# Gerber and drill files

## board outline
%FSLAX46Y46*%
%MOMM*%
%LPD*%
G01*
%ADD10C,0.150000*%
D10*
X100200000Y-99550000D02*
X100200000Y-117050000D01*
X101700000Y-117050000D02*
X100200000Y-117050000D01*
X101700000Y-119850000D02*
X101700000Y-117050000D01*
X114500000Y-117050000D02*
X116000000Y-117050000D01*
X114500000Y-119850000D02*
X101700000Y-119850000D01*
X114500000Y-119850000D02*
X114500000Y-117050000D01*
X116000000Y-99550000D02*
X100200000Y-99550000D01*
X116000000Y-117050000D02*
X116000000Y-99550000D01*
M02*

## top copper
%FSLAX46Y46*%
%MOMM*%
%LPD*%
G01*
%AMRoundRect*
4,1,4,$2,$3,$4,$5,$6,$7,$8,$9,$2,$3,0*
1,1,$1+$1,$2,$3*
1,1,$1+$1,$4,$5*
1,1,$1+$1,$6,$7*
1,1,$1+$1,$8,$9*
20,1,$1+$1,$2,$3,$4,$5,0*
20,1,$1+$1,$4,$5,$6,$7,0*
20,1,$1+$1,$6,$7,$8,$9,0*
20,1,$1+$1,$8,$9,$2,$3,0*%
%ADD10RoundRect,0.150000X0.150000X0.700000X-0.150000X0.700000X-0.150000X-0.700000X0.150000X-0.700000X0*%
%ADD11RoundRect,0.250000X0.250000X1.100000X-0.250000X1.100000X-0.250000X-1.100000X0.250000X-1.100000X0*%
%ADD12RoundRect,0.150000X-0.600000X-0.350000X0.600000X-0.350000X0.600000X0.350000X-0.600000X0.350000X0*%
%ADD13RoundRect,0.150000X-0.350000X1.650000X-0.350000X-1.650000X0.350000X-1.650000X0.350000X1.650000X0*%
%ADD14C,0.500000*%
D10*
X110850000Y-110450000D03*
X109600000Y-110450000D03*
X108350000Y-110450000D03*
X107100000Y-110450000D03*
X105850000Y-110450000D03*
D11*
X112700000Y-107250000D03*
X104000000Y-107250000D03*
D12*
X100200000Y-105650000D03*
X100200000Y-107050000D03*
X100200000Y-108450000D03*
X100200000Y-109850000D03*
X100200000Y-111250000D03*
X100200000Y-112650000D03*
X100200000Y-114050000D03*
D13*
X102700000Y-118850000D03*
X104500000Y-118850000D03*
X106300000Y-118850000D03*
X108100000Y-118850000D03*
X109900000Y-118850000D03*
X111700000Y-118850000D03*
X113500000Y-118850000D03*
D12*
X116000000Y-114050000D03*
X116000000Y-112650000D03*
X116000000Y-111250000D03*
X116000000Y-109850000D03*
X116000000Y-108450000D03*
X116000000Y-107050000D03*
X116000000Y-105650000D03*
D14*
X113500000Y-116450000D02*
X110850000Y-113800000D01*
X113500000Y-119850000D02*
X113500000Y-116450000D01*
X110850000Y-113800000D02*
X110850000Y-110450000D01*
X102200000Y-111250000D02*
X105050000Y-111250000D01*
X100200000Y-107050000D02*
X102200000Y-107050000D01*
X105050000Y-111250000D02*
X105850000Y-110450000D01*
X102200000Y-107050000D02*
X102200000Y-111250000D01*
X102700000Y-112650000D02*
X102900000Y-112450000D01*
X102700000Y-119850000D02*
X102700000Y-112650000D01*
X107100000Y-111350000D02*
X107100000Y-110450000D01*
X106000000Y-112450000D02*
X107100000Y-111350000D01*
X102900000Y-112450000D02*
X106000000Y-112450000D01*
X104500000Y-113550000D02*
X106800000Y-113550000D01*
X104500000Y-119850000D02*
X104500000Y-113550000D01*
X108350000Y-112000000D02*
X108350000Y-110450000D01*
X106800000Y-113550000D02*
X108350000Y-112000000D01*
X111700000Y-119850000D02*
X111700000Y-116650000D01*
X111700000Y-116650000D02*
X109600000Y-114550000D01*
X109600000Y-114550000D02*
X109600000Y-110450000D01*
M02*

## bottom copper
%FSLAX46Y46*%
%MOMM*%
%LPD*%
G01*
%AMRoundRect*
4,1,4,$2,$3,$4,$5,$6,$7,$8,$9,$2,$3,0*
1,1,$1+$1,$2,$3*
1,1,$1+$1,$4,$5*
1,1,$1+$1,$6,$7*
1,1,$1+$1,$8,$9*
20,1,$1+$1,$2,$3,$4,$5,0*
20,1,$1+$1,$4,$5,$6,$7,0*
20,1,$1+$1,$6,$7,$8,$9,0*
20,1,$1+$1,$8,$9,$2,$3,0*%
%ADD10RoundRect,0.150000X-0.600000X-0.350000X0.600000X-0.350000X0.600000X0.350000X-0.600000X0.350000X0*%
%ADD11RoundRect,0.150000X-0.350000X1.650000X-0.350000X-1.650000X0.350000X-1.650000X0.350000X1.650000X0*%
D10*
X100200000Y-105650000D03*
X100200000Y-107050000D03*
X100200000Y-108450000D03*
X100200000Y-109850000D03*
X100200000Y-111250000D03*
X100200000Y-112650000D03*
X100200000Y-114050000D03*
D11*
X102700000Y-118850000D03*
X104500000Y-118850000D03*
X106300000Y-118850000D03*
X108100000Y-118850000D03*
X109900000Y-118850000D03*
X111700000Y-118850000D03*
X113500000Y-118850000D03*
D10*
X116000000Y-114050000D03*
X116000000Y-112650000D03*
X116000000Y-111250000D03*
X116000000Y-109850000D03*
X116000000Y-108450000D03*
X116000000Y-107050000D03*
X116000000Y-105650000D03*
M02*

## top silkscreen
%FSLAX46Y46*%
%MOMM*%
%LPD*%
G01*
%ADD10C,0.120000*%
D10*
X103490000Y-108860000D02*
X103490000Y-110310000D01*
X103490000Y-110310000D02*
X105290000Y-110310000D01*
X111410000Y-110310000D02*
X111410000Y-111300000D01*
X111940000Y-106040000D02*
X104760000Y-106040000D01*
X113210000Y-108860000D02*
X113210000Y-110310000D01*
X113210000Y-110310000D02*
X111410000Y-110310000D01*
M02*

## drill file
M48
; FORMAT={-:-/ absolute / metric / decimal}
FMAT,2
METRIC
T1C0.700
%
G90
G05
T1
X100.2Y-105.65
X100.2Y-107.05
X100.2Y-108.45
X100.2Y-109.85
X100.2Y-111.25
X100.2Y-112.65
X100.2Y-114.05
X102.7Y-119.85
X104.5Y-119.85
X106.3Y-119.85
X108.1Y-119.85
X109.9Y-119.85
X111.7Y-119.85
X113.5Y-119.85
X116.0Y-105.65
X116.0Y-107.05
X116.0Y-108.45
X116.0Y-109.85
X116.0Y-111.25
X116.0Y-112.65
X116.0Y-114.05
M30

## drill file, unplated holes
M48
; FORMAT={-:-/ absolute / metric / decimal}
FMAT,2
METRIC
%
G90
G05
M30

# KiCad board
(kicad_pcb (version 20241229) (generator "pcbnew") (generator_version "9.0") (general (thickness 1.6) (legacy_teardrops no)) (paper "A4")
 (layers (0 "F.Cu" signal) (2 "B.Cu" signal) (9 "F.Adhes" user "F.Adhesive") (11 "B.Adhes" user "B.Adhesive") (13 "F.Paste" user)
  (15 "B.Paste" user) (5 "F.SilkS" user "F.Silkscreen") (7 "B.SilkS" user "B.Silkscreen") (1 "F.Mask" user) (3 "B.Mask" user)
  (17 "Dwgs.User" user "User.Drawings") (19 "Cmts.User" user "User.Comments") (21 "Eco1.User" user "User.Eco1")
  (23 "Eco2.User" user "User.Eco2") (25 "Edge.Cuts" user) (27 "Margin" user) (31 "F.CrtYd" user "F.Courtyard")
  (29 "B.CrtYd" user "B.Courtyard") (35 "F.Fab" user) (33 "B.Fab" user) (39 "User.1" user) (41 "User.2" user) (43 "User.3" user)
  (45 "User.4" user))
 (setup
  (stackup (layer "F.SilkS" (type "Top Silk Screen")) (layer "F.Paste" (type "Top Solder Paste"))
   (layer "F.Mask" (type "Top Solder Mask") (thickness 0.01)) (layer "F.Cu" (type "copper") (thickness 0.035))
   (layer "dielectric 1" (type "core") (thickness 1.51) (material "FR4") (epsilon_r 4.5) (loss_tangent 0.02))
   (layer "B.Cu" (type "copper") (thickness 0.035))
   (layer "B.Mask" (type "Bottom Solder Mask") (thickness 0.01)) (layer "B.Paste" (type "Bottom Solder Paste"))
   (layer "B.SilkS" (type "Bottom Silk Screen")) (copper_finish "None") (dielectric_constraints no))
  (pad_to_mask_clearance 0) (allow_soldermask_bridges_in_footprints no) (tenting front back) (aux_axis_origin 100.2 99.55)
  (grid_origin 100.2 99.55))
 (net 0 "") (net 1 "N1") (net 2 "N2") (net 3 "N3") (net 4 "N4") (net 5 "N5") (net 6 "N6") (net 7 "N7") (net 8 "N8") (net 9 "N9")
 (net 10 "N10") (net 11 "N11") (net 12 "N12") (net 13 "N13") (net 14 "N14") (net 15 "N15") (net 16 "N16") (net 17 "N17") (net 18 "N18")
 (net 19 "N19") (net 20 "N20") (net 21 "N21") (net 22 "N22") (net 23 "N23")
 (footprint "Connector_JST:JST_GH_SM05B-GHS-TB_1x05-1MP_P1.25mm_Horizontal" (layer "F.Cu") (at 108.35 108.6 180)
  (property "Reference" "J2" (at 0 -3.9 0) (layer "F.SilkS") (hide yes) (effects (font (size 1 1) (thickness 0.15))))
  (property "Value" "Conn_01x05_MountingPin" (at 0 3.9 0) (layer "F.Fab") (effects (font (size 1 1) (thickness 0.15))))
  (fp_line (start 4.86 -0.26) (end 4.86 -1.71) (stroke (width 0.12) (type solid)) (layer "F.SilkS"))
  (fp_line (start 4.86 -1.71) (end 3.06 -1.71) (stroke (width 0.12) (type solid)) (layer "F.SilkS"))
  (fp_line (start -3.06 -1.71) (end -3.06 -2.7) (stroke (width 0.12) (type solid)) (layer "F.SilkS"))
  (fp_line (start -3.59 2.56) (end 3.59 2.56) (stroke (width 0.12) (type solid)) (layer "F.SilkS"))
  (fp_line (start -4.86 -0.26) (end -4.86 -1.71) (stroke (width 0.12) (type solid)) (layer "F.SilkS"))
  (fp_line (start -4.86 -1.71) (end -3.06 -1.71) (stroke (width 0.12) (type solid)) (layer "F.SilkS"))
  (pad "1" smd roundrect (at -2.5 -1.85 180) (size 0.6 1.7) (layers "F.Cu" "F.Mask" "F.Paste") (roundrect_rratio 0.25) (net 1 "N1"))
  (pad "2" smd roundrect (at -1.25 -1.85 180) (size 0.6 1.7) (layers "F.Cu" "F.Mask" "F.Paste") (roundrect_rratio 0.25) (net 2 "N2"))
  (pad "3" smd roundrect (at 0 -1.85 180) (size 0.6 1.7) (layers "F.Cu" "F.Mask" "F.Paste") (roundrect_rratio 0.25) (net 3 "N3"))
  (pad "4" smd roundrect (at 1.25 -1.85 180) (size 0.6 1.7) (layers "F.Cu" "F.Mask" "F.Paste") (roundrect_rratio 0.25) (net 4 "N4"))
  (pad "5" smd roundrect (at 2.5 -1.85 180) (size 0.6 1.7) (layers "F.Cu" "F.Mask" "F.Paste") (roundrect_rratio 0.25) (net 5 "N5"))
  (pad "MP" smd roundrect (at -4.35 1.35 180) (size 1 2.7) (layers "F.Cu" "F.Mask" "F.Paste") (roundrect_rratio 0.25) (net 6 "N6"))
  (pad "MP" smd roundrect (at 4.35 1.35 180) (size 1 2.7) (layers "F.Cu" "F.Mask" "F.Paste") (roundrect_rratio 0.25) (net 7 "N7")))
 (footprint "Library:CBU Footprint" (layer "F.Cu") (at 100.2 99.55)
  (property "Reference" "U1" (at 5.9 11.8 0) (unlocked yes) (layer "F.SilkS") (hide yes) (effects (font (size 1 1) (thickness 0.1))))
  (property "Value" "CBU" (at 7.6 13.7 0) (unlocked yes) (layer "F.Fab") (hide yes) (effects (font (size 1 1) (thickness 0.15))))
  (fp_line (start 0 0) (end 0 17.5) (stroke (width 0.15) (type solid)) (layer "Edge.Cuts"))
  (fp_line (start 1.5 17.5) (end 0 17.5) (stroke (width 0.15) (type solid)) (layer "Edge.Cuts"))
  (fp_line (start 1.5 20.3) (end 1.5 17.5) (stroke (width 0.15) (type solid)) (layer "Edge.Cuts"))
  (fp_line (start 14.3 17.5) (end 15.8 17.5) (stroke (width 0.15) (type solid)) (layer "Edge.Cuts"))
  (fp_line (start 14.3 20.3) (end 1.5 20.3) (stroke (width 0.15) (type solid)) (layer "Edge.Cuts"))
  (fp_line (start 14.3 20.3) (end 14.3 17.5) (stroke (width 0.15) (type solid)) (layer "Edge.Cuts"))
  (fp_line (start 15.8 0) (end 0 0) (stroke (width 0.15) (type solid)) (layer "Edge.Cuts"))
  (fp_line (start 15.8 17.5) (end 15.8 0) (stroke (width 0.15) (type solid)) (layer "Edge.Cuts"))
  (pad "1" thru_hole roundrect (at 0 6.1) (size 1.5 1) (drill 0.7) (layers "*.Cu" "*.Mask") (remove_unused_layers no)
   (roundrect_rratio 0.15) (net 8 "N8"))
  (pad "2" thru_hole roundrect (at 0 7.5) (size 1.5 1) (drill 0.7) (layers "*.Cu" "*.Mask") (remove_unused_layers no)
   (roundrect_rratio 0.15) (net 5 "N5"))
  (pad "3" thru_hole roundrect (at 0 8.9) (size 1.5 1) (drill 0.7) (layers "*.Cu" "*.Mask") (remove_unused_layers no)
   (roundrect_rratio 0.15) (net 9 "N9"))
  (pad "4" thru_hole roundrect (at 0 10.3) (size 1.5 1) (drill 0.7) (layers "*.Cu" "*.Mask") (remove_unused_layers no)
   (roundrect_rratio 0.15) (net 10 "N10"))
  (pad "5" thru_hole roundrect (at 0 11.7) (size 1.5 1) (drill 0.7) (layers "*.Cu" "*.Mask") (remove_unused_layers no)
   (roundrect_rratio 0.15) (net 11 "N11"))
  (pad "6" thru_hole roundrect (at 0 13.1) (size 1.5 1) (drill 0.7) (layers "*.Cu" "*.Mask") (remove_unused_layers no)
   (roundrect_rratio 0.15) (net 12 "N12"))
  (pad "7" thru_hole roundrect (at 0 14.5) (size 1.5 1) (drill 0.7) (layers "*.Cu" "*.Mask") (remove_unused_layers no)
   (roundrect_rratio 0.15) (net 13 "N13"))
  (pad "8" thru_hole roundrect (at 2.5 20.3 270) (size 3.6 1) (drill 0.7 (offset -1 0)) (layers "*.Cu" "*.Mask") (remove_unused_layers no)
   (roundrect_rratio 0.15) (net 4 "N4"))
  (pad "9" thru_hole roundrect (at 4.3 20.3 270) (size 3.6 1) (drill 0.7 (offset -1 0)) (layers "*.Cu" "*.Mask") (remove_unused_layers no)
   (roundrect_rratio 0.15) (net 3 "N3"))
  (pad "10" thru_hole roundrect (at 6.1 20.3 270) (size 3.6 1) (drill 0.7 (offset -1 0)) (layers "*.Cu" "*.Mask") (remove_unused_layers no)
   (roundrect_rratio 0.15) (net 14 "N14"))
  (pad "11" thru_hole roundrect (at 7.9 20.3 270) (size 3.6 1) (drill 0.7 (offset -1 0)) (layers "*.Cu" "*.Mask") (remove_unused_layers no)
   (roundrect_rratio 0.15) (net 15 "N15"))
  (pad "12" thru_hole roundrect (at 9.7 20.3 270) (size 3.6 1) (drill 0.7 (offset -1 0)) (layers "*.Cu" "*.Mask") (remove_unused_layers no)
   (roundrect_rratio 0.15) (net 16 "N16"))
  (pad "13" thru_hole roundrect (at 11.5 20.3 270) (size 3.6 1) (drill 0.7 (offset -1 0)) (layers "*.Cu" "*.Mask") (remove_unused_layers no)
   (roundrect_rratio 0.15) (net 2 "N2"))
  (pad "14" thru_hole roundrect (at 13.3 20.3 270) (size 3.6 1) (drill 0.7 (offset -1 0)) (layers "*.Cu" "*.Mask") (remove_unused_layers no)
   (roundrect_rratio 0.15) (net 1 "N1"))
  (pad "15" thru_hole roundrect (at 15.8 14.5) (size 1.5 1) (drill 0.7) (layers "*.Cu" "*.Mask") (remove_unused_layers no)
   (roundrect_rratio 0.15) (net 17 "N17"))
  (pad "16" thru_hole roundrect (at 15.8 13.1) (size 1.5 1) (drill 0.7) (layers "*.Cu" "*.Mask") (remove_unused_layers no)
   (roundrect_rratio 0.15) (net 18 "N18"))
  (pad "17" thru_hole roundrect (at 15.8 11.7) (size 1.5 1) (drill 0.7) (layers "*.Cu" "*.Mask") (remove_unused_layers no)
   (roundrect_rratio 0.15) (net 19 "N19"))
  (pad "18" thru_hole roundrect (at 15.8 10.3) (size 1.5 1) (drill 0.7) (layers "*.Cu" "*.Mask") (remove_unused_layers no)
   (roundrect_rratio 0.15) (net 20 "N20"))
  (pad "19" thru_hole roundrect (at 15.8 8.9) (size 1.5 1) (drill 0.7) (layers "*.Cu" "*.Mask") (remove_unused_layers no)
   (roundrect_rratio 0.15) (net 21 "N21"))
  (pad "20" thru_hole roundrect (at 15.8 7.5) (size 1.5 1) (drill 0.7) (layers "*.Cu" "*.Mask") (remove_unused_layers no)
   (roundrect_rratio 0.15) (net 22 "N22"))
  (pad "21" thru_hole roundrect (at 15.8 6.1) (size 1.5 1) (drill 0.7) (layers "*.Cu" "*.Mask") (remove_unused_layers no)
   (roundrect_rratio 0.15) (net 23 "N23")))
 (segment (start 113.5 116.45) (end 110.85 113.8) (width 0.5) (layer "F.Cu") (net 1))
 (segment (start 113.5 119.85) (end 113.5 116.45) (width 0.5) (layer "F.Cu") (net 1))
 (segment (start 110.85 113.8) (end 110.85 110.45) (width 0.5) (layer "F.Cu") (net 1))
 (segment (start 102.2 111.25) (end 105.05 111.25) (width 0.5) (layer "F.Cu") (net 5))
 (segment (start 100.2 107.05) (end 102.2 107.05) (width 0.5) (layer "F.Cu") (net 5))
 (segment (start 105.05 111.25) (end 105.85 110.45) (width 0.5) (layer "F.Cu") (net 5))
 (segment (start 102.2 107.05) (end 102.2 111.25) (width 0.5) (layer "F.Cu") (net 5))
 (segment (start 102.7 112.65) (end 102.9 112.45) (width 0.5) (layer "F.Cu") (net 4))
 (segment (start 102.7 119.85) (end 102.7 112.65) (width 0.5) (layer "F.Cu") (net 4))
 (segment (start 107.1 111.35) (end 107.1 110.45) (width 0.5) (layer "F.Cu") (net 4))
 (segment (start 106 112.45) (end 107.1 111.35) (width 0.5) (layer "F.Cu") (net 4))
 (segment (start 102.9 112.45) (end 106 112.45) (width 0.5) (layer "F.Cu") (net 4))
 (segment (start 104.5 113.55) (end 106.8 113.55) (width 0.5) (layer "F.Cu") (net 3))
 (segment (start 104.5 119.85) (end 104.5 113.55) (width 0.5) (layer "F.Cu") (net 3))
 (segment (start 108.35 112) (end 108.35 110.45) (width 0.5) (layer "F.Cu") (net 3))
 (segment (start 106.8 113.55) (end 108.35 112) (width 0.5) (layer "F.Cu") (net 3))
 (segment (start 111.7 119.85) (end 111.7 116.65) (width 0.5) (layer "F.Cu") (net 2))
 (segment (start 111.7 116.65) (end 109.6 114.55) (width 0.5) (layer "F.Cu") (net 2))
 (segment (start 109.6 114.55) (end 109.6 110.45) (width 0.5) (layer "F.Cu") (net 2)))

